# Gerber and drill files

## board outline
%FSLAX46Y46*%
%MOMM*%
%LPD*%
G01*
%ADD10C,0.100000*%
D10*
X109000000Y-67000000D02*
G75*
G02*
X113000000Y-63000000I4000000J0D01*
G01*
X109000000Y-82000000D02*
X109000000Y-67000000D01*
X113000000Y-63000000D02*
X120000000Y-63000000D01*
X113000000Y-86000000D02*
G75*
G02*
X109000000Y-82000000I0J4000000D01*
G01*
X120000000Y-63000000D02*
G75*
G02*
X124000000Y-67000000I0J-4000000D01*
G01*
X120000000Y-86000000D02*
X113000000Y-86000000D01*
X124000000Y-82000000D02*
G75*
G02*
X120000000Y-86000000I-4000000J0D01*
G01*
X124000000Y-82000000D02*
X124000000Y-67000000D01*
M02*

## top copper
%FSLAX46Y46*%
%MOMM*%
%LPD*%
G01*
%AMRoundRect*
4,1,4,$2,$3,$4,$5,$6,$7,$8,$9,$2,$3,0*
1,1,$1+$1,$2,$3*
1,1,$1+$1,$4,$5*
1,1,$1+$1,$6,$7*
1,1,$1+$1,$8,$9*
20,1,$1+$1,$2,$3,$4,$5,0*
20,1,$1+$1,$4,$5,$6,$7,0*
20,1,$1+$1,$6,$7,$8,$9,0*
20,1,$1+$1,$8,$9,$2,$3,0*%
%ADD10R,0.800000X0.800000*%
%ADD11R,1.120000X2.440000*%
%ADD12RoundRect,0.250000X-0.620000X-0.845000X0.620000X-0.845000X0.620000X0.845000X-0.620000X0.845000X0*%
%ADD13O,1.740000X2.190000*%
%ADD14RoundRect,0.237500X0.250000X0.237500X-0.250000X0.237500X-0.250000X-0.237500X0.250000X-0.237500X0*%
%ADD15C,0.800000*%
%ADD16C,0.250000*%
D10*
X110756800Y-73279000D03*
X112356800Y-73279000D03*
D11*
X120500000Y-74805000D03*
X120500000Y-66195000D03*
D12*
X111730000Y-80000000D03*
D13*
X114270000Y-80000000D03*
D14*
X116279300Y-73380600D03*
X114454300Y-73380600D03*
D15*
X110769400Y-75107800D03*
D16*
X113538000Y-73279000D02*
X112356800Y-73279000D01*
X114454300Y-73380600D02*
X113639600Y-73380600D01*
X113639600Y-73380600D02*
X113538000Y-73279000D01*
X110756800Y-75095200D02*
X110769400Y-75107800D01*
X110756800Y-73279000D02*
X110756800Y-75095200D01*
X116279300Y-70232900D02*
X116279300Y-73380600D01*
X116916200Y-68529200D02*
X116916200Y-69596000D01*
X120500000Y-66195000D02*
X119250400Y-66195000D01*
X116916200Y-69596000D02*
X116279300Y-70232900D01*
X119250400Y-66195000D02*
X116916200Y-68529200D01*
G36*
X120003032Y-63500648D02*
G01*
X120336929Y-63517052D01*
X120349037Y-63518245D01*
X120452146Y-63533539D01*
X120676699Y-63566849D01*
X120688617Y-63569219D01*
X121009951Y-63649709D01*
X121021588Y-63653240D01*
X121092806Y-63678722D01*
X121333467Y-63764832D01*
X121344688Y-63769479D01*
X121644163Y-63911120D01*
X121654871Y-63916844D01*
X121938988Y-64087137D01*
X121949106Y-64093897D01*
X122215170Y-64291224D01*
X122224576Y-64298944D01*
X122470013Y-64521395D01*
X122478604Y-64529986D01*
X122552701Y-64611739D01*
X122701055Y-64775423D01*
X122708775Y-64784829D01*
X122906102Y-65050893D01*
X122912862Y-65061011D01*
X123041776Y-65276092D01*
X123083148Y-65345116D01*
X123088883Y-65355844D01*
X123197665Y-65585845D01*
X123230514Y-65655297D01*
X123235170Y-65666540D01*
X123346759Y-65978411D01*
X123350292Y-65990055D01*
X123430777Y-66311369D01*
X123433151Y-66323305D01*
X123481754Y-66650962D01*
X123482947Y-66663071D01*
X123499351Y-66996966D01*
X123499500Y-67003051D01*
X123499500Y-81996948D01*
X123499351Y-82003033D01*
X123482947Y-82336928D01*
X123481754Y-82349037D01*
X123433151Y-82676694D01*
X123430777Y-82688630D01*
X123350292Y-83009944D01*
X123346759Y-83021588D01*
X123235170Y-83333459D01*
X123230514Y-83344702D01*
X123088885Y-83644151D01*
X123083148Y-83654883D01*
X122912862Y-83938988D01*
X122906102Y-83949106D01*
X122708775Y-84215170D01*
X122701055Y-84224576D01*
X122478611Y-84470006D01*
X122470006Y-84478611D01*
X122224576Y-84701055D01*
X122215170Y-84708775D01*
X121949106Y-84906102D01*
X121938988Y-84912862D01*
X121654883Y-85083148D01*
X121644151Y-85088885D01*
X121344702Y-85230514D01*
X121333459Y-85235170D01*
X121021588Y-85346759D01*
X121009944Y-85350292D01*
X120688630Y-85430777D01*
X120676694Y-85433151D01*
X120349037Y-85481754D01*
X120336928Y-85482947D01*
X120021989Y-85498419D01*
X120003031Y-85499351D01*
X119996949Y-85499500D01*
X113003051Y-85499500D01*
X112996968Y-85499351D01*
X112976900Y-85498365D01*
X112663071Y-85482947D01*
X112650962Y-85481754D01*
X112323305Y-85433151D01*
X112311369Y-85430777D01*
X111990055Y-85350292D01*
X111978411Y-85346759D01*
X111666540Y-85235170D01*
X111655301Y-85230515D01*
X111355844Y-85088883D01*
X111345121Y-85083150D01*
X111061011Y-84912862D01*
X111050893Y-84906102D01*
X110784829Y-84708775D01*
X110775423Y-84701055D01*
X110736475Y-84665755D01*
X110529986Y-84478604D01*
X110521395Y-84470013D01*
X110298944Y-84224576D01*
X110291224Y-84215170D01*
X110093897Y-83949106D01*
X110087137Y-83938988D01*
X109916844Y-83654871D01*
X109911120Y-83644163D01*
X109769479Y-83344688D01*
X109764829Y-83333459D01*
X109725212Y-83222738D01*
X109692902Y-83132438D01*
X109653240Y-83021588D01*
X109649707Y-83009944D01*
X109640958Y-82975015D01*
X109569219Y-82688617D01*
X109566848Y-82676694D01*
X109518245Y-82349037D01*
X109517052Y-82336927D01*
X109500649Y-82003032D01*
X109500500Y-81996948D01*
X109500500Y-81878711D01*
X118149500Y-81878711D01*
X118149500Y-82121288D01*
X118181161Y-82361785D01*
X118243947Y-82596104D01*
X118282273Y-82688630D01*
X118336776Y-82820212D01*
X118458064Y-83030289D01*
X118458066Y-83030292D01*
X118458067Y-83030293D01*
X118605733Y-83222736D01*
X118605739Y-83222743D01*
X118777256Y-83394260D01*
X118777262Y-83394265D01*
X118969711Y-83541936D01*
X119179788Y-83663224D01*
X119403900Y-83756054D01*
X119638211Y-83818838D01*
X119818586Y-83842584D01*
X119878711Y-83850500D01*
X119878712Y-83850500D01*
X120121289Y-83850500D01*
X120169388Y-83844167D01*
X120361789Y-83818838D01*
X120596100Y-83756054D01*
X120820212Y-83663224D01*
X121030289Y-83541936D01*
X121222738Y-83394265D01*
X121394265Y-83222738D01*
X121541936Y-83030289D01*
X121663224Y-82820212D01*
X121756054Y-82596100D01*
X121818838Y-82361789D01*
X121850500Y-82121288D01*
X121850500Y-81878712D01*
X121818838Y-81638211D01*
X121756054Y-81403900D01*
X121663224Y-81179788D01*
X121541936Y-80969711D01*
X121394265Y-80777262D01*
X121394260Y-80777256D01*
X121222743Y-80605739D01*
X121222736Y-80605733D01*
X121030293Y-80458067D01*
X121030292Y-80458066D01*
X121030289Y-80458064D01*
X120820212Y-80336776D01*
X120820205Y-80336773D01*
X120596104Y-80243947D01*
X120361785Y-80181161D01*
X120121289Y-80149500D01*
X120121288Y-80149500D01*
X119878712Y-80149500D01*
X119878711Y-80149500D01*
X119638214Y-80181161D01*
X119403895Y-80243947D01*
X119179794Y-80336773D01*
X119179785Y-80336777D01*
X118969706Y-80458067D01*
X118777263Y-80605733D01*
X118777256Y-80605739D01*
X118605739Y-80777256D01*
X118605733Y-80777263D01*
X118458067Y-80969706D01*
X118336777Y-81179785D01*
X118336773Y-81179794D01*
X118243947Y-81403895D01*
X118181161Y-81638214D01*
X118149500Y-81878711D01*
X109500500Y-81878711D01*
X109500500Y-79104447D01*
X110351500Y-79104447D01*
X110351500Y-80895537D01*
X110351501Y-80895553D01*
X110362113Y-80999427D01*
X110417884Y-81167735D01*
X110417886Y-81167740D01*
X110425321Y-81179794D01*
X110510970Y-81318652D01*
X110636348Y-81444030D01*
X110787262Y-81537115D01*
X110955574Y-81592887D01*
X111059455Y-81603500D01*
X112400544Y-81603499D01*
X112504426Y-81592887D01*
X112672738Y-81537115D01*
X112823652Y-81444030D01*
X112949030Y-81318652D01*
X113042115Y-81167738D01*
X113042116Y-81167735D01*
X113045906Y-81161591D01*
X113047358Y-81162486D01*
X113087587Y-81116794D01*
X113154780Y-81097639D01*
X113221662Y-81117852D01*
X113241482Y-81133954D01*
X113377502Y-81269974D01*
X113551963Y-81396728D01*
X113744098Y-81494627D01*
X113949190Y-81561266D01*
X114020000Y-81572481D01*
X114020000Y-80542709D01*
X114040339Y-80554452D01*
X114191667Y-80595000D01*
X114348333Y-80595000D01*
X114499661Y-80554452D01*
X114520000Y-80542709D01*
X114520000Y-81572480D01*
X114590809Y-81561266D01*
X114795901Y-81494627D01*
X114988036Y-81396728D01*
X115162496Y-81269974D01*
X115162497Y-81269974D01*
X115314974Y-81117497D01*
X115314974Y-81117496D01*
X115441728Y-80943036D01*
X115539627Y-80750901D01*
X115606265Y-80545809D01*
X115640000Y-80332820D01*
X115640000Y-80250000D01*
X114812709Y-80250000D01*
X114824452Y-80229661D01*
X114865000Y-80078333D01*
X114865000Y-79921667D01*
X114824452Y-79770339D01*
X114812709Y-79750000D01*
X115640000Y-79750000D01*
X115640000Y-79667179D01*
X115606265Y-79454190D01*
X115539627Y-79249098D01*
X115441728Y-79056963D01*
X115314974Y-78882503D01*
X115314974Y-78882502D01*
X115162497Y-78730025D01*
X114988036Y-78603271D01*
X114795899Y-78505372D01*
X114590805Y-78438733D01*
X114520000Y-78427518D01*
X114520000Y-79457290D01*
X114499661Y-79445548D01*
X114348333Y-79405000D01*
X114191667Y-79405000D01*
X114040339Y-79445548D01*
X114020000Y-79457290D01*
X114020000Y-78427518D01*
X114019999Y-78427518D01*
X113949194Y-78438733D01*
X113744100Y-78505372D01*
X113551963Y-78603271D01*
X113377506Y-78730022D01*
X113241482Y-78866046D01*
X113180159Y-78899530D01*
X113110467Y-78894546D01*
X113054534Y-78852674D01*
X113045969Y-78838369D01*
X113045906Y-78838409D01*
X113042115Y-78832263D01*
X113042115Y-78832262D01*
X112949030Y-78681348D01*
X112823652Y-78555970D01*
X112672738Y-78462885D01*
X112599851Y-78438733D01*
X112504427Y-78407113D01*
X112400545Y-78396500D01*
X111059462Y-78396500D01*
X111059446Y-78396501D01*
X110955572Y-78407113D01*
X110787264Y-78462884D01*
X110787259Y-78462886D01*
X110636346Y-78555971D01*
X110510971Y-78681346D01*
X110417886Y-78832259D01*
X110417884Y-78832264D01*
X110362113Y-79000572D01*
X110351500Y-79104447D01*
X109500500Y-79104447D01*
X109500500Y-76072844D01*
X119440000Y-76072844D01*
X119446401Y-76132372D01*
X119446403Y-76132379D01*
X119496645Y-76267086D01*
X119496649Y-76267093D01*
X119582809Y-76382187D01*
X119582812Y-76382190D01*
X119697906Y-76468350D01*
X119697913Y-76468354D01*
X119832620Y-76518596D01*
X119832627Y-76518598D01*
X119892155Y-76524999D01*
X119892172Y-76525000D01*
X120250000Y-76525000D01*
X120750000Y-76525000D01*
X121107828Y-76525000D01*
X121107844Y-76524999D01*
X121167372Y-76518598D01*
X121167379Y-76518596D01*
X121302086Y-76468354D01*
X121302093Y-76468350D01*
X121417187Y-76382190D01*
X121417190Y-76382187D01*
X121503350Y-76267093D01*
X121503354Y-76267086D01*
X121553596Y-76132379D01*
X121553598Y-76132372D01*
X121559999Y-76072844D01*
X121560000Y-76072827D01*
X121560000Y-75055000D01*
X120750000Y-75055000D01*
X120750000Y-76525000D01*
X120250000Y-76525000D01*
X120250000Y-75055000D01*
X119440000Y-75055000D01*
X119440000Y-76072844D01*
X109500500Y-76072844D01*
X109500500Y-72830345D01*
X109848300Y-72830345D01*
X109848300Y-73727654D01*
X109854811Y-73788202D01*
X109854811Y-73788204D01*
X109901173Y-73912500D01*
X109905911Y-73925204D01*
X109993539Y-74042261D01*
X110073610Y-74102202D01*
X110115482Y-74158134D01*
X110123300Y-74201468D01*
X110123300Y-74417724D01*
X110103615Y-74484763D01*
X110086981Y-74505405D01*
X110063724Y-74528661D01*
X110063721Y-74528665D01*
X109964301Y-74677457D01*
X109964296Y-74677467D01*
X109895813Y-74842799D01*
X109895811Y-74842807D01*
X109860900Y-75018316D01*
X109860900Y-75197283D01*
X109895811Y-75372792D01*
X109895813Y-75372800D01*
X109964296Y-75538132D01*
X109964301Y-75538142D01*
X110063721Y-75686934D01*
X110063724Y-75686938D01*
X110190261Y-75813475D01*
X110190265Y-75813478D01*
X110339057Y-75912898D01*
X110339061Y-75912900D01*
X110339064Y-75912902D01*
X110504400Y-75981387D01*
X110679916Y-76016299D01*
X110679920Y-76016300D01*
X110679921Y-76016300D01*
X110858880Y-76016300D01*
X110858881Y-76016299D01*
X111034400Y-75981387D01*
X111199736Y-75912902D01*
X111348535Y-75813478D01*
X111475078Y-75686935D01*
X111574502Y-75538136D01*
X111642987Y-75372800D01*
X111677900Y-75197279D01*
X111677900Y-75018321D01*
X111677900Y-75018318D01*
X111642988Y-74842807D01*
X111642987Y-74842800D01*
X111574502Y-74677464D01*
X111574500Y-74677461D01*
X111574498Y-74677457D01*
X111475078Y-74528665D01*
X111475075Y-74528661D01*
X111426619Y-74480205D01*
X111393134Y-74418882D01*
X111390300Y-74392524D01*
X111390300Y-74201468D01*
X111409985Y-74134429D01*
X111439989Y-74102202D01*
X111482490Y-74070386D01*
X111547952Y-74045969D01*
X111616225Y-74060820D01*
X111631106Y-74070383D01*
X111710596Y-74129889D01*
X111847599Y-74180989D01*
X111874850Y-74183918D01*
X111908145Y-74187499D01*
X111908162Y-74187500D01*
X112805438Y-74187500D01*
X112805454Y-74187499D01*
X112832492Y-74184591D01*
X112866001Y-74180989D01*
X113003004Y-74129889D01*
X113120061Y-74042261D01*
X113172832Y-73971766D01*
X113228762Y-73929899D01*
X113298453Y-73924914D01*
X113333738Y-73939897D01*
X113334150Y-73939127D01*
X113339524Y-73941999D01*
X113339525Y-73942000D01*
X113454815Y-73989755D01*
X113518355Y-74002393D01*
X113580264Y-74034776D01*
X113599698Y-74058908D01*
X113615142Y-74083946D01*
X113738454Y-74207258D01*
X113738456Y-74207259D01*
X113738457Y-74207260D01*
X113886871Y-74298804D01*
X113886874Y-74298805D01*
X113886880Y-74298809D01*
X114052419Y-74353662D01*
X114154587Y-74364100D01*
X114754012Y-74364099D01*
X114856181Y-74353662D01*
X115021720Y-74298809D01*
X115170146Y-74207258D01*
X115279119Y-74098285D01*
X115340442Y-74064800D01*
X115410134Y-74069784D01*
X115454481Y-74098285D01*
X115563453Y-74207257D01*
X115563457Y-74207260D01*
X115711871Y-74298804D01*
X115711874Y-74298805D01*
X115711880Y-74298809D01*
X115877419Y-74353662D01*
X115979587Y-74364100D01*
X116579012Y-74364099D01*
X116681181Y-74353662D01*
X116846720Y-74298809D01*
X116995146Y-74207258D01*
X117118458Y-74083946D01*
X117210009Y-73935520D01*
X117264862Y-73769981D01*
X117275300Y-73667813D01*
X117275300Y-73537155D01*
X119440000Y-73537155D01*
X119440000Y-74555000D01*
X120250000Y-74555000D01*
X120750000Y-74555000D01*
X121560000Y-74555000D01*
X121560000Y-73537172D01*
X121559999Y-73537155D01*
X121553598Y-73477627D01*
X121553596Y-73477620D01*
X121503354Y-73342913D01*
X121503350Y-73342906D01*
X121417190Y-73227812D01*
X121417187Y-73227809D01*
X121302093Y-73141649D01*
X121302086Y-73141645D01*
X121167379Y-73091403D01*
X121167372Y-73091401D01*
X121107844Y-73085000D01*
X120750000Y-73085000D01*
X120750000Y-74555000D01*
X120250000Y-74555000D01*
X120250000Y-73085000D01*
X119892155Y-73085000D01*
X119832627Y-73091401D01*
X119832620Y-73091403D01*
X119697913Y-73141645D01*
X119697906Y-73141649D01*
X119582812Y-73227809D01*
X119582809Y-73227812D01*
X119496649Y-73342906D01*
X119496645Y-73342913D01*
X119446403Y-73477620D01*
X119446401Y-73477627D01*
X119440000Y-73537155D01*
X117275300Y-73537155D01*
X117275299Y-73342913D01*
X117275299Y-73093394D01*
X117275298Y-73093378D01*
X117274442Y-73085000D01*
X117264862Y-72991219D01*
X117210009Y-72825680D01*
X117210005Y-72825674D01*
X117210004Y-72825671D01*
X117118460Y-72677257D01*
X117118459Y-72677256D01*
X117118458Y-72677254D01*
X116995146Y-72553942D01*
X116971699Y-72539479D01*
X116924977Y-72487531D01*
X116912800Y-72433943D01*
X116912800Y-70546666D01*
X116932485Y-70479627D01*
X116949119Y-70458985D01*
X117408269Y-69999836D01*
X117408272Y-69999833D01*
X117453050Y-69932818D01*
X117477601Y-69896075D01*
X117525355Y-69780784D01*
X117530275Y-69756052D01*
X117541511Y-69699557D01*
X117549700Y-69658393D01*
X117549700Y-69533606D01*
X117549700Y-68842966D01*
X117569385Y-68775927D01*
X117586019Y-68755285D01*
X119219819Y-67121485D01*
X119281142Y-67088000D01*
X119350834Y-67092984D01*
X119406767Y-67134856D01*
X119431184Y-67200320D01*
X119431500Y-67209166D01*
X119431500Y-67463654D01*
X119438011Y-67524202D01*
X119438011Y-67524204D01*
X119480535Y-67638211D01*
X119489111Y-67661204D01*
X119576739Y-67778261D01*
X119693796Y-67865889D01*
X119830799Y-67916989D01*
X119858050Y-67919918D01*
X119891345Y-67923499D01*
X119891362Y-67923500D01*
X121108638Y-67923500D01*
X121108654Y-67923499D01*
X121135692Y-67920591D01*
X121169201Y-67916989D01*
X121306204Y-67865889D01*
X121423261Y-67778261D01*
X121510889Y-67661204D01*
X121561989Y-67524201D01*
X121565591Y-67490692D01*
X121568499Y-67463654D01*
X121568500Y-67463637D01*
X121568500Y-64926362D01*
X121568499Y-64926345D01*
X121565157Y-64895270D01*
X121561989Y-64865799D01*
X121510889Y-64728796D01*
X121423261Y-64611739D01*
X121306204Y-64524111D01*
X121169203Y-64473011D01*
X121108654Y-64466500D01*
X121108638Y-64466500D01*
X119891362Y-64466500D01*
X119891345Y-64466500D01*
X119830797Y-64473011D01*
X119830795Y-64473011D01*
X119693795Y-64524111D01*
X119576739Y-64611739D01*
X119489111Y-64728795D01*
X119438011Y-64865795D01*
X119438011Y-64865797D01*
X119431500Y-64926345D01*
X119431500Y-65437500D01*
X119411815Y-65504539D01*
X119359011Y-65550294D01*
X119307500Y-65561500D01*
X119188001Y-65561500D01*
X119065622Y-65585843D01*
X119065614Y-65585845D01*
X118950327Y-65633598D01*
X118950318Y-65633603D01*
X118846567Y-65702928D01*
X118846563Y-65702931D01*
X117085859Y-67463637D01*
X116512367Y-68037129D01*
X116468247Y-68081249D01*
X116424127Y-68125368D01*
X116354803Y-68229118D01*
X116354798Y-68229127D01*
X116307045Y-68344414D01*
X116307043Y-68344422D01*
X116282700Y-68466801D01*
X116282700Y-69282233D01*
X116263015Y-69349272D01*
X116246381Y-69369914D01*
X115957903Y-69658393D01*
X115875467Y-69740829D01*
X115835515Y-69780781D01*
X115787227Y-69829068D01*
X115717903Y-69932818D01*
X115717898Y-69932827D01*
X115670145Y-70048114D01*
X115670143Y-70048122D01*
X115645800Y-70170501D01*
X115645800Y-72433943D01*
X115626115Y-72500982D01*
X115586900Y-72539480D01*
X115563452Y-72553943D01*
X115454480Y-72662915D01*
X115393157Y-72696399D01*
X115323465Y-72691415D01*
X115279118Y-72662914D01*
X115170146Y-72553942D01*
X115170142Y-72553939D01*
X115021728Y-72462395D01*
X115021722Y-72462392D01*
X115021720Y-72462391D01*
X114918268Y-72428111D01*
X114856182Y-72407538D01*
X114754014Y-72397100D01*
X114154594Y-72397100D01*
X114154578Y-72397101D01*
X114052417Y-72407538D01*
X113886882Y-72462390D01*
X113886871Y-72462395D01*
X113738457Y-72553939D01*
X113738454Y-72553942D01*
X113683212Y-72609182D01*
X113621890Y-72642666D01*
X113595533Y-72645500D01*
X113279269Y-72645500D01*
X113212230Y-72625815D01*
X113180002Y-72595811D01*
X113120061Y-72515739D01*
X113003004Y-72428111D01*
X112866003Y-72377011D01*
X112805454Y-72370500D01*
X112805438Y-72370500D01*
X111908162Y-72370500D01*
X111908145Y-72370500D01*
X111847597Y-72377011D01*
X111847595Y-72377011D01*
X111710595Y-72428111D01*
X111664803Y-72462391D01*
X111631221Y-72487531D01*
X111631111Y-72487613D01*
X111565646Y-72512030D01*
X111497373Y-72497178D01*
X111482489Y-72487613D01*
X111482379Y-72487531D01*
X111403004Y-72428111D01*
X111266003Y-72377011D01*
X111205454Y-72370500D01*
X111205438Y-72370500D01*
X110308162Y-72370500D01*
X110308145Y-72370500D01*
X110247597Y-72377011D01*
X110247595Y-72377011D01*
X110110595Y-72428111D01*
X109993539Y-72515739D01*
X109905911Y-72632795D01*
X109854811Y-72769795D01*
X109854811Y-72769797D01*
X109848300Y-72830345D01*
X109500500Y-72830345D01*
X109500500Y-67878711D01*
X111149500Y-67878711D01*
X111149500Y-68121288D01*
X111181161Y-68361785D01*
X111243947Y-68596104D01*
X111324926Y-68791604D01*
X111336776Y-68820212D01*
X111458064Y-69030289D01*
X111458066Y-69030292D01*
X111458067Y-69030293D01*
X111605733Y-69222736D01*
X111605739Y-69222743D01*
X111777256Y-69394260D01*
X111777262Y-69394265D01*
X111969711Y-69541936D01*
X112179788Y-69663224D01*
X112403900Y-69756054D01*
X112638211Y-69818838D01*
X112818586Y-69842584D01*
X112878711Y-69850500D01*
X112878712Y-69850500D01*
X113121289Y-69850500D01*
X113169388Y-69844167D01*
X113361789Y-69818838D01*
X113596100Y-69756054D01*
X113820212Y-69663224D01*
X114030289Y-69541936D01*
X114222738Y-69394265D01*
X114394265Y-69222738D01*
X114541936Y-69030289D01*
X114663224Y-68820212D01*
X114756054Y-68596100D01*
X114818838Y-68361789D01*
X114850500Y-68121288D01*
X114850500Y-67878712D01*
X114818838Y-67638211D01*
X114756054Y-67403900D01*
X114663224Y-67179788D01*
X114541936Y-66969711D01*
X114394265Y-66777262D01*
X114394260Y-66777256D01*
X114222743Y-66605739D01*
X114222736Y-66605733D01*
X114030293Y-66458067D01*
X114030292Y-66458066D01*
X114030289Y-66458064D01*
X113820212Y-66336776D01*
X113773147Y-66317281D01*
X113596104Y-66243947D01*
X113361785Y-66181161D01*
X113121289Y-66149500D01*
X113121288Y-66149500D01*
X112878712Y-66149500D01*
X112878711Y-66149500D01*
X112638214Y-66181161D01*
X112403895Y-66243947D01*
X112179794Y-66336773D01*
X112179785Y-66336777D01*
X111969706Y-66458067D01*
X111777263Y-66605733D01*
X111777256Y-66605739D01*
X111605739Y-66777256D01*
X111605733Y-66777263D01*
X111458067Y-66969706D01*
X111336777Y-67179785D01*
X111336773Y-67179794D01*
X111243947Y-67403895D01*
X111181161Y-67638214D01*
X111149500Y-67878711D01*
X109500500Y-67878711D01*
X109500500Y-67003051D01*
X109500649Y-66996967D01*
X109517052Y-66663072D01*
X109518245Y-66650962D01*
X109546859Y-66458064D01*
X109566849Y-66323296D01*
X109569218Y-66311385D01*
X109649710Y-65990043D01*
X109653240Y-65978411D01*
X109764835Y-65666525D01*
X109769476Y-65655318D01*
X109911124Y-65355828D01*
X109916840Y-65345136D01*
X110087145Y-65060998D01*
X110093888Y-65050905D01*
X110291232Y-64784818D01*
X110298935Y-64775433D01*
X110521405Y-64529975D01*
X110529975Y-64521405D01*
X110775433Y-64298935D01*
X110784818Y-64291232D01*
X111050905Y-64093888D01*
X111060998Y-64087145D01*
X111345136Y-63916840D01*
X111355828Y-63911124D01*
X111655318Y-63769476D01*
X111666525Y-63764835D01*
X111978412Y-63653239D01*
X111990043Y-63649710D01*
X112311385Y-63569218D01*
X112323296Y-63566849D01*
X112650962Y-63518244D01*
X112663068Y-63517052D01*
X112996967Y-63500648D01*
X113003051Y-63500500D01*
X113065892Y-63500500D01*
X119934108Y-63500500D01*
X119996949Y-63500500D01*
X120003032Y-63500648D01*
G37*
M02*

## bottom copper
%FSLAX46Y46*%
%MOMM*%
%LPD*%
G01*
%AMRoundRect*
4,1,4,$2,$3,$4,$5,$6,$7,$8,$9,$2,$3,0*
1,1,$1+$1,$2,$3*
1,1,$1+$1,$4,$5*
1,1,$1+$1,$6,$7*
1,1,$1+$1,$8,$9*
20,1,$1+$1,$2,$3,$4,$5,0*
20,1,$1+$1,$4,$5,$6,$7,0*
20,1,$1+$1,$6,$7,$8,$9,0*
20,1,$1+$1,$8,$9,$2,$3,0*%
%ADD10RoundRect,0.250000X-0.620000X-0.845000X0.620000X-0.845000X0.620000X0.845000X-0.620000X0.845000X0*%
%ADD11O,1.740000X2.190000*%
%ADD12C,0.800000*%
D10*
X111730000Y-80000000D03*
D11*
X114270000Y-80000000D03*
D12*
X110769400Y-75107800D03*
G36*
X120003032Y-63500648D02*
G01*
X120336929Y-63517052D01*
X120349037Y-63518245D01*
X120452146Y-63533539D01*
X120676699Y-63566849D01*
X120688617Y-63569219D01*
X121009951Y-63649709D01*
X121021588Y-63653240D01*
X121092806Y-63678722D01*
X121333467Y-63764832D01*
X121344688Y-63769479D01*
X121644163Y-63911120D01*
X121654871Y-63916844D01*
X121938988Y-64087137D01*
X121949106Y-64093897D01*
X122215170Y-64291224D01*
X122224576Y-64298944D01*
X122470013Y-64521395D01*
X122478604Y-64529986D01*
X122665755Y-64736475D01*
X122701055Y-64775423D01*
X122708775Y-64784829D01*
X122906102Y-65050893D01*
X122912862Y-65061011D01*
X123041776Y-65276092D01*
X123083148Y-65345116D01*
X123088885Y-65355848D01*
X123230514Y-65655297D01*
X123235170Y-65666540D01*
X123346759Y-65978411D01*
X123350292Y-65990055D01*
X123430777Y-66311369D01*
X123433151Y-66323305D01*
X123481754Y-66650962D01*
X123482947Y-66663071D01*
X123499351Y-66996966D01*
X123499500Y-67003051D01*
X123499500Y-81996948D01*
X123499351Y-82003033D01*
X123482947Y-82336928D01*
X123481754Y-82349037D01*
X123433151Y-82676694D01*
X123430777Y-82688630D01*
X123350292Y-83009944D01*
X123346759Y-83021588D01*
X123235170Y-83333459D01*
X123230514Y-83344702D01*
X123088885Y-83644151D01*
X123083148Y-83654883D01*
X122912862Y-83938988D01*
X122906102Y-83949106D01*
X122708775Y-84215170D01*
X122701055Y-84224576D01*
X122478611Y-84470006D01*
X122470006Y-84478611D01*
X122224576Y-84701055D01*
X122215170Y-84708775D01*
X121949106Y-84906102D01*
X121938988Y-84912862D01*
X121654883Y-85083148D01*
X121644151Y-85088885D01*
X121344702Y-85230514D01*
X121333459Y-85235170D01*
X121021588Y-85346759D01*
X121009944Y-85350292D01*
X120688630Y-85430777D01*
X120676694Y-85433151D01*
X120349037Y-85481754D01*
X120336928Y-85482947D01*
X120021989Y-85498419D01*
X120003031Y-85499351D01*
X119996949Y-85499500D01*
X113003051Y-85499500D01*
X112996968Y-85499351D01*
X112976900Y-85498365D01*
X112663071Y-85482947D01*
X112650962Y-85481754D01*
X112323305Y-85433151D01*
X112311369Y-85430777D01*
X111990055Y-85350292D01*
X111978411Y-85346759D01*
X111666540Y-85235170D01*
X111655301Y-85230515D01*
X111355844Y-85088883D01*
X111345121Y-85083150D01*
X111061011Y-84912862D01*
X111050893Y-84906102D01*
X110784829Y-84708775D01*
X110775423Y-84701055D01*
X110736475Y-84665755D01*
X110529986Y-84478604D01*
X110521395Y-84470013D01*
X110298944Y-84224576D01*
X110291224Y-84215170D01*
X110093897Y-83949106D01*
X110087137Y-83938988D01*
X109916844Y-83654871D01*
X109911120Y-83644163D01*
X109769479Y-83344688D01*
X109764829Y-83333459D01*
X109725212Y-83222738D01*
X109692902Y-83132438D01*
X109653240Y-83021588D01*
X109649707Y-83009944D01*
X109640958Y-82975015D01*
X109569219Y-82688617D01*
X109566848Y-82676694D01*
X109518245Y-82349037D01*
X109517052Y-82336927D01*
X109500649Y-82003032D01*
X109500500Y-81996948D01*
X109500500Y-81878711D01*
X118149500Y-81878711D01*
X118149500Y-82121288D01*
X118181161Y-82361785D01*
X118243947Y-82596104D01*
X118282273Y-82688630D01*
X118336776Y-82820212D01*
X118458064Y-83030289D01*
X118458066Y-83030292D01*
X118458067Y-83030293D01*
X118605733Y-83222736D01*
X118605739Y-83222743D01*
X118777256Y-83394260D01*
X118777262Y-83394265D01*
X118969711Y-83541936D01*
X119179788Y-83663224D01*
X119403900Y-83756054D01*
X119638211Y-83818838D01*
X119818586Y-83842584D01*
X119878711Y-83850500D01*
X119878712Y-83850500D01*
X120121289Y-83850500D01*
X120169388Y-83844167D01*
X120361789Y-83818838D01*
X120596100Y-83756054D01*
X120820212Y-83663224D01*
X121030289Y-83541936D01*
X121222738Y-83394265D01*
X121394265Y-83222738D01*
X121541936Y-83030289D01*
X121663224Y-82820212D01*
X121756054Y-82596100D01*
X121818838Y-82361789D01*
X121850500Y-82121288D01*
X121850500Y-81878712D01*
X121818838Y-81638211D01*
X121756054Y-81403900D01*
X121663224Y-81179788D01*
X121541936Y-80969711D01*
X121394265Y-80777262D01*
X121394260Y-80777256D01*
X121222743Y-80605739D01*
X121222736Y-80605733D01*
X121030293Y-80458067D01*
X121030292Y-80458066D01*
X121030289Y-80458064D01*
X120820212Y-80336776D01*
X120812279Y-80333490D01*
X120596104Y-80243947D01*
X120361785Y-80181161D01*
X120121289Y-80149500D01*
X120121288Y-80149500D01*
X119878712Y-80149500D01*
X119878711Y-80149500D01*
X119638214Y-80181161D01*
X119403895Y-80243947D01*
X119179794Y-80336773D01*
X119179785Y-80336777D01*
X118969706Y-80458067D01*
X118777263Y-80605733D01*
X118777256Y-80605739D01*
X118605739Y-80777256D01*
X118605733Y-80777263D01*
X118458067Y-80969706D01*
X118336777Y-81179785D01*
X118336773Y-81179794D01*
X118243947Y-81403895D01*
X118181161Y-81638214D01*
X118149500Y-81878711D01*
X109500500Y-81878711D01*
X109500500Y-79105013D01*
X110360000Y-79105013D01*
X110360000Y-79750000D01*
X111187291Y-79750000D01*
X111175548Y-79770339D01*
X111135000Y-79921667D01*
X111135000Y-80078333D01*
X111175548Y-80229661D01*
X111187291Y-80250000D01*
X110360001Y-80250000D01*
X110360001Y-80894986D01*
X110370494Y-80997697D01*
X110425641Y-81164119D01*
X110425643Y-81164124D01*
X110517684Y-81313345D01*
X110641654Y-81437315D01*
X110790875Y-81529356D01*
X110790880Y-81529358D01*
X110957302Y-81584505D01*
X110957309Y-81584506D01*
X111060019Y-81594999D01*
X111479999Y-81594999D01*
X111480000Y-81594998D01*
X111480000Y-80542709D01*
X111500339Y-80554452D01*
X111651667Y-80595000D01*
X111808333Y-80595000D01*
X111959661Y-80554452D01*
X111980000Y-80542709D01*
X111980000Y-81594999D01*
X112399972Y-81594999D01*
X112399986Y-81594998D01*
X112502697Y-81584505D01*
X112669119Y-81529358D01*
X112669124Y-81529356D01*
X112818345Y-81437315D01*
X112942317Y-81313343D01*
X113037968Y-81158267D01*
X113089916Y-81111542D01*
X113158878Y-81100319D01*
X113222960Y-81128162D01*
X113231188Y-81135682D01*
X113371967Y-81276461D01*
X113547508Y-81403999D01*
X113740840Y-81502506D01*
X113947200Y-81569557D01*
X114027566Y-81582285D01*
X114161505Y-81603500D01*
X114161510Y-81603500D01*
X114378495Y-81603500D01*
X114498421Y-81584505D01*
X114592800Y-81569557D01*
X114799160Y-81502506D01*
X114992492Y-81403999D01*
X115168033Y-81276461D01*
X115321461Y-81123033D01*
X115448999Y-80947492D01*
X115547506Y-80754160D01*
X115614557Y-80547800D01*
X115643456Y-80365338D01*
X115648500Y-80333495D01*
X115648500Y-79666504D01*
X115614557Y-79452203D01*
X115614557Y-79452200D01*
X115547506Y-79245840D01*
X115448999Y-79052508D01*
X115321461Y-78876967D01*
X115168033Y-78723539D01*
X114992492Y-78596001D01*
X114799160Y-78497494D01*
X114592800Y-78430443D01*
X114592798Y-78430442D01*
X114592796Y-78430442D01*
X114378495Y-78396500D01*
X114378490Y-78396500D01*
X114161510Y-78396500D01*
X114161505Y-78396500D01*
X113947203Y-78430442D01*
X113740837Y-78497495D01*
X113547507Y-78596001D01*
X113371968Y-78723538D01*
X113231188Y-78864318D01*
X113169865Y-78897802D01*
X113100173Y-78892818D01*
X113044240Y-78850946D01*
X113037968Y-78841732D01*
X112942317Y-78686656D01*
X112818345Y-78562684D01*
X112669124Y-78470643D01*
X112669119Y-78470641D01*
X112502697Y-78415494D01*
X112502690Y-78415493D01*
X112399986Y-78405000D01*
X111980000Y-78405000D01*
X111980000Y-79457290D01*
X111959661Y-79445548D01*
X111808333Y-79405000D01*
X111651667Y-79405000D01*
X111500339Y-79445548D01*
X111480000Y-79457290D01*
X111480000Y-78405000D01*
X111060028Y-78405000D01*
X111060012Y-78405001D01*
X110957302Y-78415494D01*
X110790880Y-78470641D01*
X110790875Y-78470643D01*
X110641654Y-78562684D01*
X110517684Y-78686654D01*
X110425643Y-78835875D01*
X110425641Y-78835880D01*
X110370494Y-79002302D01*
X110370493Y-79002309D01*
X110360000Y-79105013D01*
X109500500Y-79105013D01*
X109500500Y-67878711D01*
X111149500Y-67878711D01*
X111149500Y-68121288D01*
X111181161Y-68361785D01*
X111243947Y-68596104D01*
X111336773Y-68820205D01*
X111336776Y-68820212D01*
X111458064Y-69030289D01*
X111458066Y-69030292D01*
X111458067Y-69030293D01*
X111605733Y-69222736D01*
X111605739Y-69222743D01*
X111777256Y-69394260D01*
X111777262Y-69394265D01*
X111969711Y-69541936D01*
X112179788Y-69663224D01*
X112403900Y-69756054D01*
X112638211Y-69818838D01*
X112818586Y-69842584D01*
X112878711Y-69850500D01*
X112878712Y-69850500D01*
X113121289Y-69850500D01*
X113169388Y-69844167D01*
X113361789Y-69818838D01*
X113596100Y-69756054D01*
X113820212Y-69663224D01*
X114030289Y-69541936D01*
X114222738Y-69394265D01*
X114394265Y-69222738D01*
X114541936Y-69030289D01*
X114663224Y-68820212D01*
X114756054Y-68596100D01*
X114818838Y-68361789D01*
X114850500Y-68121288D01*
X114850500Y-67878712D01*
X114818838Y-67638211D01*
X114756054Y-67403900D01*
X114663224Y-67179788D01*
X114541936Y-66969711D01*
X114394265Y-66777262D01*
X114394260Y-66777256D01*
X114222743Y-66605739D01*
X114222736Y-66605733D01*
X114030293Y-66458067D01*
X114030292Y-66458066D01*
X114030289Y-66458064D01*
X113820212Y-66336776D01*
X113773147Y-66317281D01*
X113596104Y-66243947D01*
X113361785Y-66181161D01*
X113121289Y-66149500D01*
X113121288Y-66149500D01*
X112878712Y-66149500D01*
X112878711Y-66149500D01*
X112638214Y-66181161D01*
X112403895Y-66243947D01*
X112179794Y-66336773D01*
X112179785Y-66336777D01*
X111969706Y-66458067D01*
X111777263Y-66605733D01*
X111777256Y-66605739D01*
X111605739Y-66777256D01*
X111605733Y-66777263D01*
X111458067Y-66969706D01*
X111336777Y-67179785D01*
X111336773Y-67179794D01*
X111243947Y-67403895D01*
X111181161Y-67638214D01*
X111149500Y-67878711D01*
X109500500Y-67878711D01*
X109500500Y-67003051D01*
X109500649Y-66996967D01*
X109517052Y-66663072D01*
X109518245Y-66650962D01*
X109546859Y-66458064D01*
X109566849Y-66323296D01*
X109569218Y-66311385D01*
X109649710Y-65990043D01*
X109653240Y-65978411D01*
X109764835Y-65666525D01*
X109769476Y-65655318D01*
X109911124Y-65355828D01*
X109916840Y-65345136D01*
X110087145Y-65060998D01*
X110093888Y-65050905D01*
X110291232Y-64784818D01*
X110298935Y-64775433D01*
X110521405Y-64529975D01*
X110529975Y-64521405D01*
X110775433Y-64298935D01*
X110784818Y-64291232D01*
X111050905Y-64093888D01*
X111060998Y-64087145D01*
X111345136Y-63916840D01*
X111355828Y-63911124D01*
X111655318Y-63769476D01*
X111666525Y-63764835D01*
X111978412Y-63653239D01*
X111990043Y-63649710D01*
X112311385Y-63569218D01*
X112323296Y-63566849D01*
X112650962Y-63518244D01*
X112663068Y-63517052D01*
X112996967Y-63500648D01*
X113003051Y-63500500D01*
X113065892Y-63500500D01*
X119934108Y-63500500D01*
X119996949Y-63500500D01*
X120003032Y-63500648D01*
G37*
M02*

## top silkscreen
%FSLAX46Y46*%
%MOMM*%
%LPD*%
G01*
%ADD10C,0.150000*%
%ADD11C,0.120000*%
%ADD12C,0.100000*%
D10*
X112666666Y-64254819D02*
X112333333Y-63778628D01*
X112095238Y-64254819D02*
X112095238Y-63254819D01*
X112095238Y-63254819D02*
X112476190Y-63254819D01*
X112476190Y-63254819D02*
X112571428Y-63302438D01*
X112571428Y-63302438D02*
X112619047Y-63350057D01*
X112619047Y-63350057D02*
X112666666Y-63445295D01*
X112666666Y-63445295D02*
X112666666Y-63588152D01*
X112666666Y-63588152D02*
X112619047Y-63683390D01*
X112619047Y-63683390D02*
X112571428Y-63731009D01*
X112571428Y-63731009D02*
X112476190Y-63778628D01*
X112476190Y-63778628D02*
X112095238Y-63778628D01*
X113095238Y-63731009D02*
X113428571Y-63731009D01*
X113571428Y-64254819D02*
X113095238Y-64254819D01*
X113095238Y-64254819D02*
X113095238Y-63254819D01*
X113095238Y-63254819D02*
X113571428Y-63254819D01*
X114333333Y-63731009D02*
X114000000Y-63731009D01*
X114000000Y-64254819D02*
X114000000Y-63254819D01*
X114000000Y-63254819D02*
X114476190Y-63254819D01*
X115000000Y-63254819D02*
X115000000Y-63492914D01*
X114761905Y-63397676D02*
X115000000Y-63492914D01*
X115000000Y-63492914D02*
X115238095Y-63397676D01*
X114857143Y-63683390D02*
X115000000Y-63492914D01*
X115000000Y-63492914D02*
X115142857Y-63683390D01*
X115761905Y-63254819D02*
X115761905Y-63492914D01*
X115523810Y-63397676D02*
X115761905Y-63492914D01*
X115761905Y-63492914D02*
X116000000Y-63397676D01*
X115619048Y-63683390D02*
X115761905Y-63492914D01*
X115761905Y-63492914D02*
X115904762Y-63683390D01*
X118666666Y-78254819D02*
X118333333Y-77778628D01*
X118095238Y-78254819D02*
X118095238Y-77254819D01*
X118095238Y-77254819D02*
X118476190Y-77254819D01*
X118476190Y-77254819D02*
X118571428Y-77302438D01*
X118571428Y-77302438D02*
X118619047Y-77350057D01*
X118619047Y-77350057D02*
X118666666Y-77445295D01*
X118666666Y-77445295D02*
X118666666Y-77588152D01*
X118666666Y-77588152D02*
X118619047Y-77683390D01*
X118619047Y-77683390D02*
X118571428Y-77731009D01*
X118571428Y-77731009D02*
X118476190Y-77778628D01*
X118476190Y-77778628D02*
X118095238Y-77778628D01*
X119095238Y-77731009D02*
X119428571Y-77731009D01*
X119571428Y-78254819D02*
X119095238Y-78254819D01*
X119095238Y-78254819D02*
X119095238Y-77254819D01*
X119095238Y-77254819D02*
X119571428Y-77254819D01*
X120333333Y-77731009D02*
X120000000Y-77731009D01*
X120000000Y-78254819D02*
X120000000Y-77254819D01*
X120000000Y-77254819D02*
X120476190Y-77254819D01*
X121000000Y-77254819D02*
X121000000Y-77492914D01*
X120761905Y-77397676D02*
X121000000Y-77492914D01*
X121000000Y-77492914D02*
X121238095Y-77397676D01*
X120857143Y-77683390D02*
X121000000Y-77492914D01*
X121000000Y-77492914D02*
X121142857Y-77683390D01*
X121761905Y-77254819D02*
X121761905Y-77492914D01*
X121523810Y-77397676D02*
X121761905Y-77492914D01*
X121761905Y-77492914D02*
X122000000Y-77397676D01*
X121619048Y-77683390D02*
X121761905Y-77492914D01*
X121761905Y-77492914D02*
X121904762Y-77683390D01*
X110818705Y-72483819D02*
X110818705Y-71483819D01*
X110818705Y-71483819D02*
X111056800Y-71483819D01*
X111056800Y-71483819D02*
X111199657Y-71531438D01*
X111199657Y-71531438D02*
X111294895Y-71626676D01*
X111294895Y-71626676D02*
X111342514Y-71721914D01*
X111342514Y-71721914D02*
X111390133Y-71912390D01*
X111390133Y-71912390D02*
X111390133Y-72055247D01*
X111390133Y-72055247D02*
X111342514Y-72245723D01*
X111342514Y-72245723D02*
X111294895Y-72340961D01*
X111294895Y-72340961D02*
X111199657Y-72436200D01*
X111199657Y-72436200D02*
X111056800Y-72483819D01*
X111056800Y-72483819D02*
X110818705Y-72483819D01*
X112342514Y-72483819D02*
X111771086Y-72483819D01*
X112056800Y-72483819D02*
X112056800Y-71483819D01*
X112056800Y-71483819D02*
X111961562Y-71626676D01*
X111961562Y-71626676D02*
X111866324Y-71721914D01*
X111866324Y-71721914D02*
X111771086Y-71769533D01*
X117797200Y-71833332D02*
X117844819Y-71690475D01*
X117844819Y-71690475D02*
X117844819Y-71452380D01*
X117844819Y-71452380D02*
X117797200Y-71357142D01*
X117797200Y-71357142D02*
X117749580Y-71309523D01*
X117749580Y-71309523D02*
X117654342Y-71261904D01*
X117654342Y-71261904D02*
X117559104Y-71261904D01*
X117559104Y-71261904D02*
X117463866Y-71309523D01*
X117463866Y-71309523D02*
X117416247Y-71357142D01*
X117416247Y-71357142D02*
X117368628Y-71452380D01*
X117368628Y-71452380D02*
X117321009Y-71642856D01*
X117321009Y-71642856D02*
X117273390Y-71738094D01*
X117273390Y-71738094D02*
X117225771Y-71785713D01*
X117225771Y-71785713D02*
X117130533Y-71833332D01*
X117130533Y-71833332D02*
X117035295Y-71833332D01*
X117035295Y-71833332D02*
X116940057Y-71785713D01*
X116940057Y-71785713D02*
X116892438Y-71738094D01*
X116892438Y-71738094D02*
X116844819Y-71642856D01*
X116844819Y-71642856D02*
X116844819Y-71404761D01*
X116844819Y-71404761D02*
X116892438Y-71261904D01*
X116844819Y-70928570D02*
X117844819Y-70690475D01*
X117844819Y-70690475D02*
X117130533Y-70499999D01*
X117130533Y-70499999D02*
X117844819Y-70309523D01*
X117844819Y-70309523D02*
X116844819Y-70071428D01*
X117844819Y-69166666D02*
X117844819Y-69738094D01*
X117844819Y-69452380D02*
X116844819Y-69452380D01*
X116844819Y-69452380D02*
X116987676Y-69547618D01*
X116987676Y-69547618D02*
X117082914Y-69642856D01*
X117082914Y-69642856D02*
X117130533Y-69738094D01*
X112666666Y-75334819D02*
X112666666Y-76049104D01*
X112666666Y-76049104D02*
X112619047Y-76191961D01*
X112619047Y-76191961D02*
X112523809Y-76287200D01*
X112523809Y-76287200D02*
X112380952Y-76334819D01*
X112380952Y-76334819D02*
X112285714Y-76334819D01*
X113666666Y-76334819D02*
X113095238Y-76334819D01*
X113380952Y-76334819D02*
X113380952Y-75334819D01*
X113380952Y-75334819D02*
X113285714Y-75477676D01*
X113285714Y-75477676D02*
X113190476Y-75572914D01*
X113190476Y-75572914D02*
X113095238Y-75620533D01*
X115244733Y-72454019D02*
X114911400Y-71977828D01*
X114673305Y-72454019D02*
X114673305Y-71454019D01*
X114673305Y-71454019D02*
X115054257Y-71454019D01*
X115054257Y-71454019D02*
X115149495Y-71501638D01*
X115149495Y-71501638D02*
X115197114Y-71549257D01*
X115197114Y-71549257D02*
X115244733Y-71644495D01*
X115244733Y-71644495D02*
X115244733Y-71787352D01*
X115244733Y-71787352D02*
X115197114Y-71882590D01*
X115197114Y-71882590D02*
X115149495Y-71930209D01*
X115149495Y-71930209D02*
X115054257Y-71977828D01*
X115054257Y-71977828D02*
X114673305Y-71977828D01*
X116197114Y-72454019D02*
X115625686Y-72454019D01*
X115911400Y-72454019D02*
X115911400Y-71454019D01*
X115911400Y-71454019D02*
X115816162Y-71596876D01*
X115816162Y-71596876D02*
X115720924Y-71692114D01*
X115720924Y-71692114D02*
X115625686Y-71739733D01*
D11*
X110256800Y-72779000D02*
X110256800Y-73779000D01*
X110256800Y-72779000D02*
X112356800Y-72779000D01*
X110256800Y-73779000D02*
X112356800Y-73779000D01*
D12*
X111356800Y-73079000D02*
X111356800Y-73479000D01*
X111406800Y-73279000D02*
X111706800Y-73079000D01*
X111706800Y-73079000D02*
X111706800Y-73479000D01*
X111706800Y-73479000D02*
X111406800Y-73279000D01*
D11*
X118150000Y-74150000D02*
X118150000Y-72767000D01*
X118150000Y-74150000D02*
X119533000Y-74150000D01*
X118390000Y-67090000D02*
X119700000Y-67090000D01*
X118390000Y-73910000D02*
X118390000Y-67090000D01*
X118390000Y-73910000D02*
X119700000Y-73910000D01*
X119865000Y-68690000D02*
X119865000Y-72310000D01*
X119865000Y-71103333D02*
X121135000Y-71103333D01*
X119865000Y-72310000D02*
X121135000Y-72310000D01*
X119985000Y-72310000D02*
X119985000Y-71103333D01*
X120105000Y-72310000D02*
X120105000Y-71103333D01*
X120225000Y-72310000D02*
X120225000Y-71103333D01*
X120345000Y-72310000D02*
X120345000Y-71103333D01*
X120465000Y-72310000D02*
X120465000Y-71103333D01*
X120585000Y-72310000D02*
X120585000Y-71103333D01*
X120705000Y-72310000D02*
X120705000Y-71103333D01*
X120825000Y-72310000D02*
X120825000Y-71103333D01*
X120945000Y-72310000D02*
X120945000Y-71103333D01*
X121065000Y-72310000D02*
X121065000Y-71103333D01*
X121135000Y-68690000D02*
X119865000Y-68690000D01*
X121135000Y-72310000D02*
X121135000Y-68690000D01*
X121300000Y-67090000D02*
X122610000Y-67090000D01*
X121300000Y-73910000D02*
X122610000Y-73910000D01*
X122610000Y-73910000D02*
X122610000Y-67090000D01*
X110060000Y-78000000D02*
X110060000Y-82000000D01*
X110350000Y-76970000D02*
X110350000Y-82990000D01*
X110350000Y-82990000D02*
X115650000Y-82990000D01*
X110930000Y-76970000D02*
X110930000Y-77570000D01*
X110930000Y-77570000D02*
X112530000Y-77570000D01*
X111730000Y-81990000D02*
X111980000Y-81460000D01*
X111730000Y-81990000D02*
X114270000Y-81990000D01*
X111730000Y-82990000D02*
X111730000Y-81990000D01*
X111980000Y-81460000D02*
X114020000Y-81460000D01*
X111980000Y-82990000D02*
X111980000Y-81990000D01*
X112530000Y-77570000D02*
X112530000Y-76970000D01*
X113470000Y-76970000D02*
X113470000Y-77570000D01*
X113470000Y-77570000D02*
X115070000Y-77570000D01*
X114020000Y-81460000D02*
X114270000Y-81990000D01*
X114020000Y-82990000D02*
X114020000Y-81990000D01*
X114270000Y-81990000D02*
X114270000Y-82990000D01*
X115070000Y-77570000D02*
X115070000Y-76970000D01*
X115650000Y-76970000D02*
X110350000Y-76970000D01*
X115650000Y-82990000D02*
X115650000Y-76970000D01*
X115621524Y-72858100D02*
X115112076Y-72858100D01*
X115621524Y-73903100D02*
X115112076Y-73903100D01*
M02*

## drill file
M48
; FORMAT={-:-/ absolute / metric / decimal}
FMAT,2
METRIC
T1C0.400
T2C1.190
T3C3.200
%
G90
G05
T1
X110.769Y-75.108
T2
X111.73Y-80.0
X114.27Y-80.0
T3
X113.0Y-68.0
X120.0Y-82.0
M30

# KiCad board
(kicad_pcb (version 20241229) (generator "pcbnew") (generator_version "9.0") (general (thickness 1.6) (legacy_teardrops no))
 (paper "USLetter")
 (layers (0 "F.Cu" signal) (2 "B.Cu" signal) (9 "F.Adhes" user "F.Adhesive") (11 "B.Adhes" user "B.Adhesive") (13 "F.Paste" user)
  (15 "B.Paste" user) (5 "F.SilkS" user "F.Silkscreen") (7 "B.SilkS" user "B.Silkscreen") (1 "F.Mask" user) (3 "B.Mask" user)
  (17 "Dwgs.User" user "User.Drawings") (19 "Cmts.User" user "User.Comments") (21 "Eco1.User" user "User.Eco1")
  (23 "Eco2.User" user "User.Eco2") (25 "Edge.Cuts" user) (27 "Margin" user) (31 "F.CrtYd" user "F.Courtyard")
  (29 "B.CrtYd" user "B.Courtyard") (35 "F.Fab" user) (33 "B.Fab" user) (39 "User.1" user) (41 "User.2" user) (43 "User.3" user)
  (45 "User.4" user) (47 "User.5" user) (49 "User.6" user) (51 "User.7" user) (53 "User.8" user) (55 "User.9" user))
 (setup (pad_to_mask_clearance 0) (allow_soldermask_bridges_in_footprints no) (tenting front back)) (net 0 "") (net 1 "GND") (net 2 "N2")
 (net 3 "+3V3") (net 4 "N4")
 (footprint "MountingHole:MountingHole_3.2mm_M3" (layer "F.Cu") (at 113 68)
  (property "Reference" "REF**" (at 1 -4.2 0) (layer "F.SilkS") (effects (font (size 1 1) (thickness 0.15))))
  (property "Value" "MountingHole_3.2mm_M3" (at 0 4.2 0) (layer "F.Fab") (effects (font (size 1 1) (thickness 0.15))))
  (pad "" np_thru_hole circle (at 0 0) (size 3.2 3.2) (drill 3.2) (layers "*.Cu" "*.Mask")))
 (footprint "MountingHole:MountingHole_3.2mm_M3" (layer "F.Cu") (at 120 82)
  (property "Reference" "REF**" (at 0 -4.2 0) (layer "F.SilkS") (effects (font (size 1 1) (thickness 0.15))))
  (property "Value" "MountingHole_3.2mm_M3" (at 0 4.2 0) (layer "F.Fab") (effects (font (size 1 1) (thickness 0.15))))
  (pad "" np_thru_hole circle (at 0 0) (size 3.2 3.2) (drill 3.2) (layers "*.Cu" "*.Mask")))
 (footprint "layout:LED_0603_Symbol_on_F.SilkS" (layer "F.Cu") (at 111.5568 73.279)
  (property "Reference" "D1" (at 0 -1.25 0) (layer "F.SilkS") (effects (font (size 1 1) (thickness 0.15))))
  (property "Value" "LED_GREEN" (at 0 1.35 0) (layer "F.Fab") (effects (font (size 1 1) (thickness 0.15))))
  (fp_line (start -1.3 -0.5) (end -1.3 0.5) (stroke (width 0.12) (type solid)) (layer "F.SilkS"))
  (fp_line (start -1.3 -0.5) (end 0.8 -0.5) (stroke (width 0.12) (type solid)) (layer "F.SilkS"))
  (fp_line (start -1.3 0.5) (end 0.8 0.5) (stroke (width 0.12) (type solid)) (layer "F.SilkS"))
  (fp_line (start -0.2 -0.2) (end -0.2 0.2) (stroke (width 0.1) (type solid)) (layer "F.SilkS"))
  (fp_line (start -0.15 0) (end 0.15 -0.2) (stroke (width 0.1) (type solid)) (layer "F.SilkS"))
  (fp_line (start 0.15 -0.2) (end 0.15 0.2) (stroke (width 0.1) (type solid)) (layer "F.SilkS"))
  (fp_line (start 0.15 0.2) (end -0.15 0) (stroke (width 0.1) (type solid)) (layer "F.SilkS"))
  (pad "1" smd rect (at -0.8 0 180) (size 0.8 0.8) (layers "F.Cu" "F.Mask" "F.Paste") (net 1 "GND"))
  (pad "2" smd rect (at 0.8 0 180) (size 0.8 0.8) (layers "F.Cu" "F.Mask" "F.Paste") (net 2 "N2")))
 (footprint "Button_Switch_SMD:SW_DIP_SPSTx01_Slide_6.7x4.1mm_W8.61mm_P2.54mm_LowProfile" (layer "F.Cu") (at 120.5 70.5 90)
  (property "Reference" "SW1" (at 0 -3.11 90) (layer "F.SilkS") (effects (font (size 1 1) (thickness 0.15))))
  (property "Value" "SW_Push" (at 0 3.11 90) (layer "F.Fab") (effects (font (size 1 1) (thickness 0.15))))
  (fp_line (start -3.65 -2.35) (end -2.267 -2.35) (stroke (width 0.12) (type solid)) (layer "F.SilkS"))
  (fp_line (start -3.65 -2.35) (end -3.65 -0.967) (stroke (width 0.12) (type solid)) (layer "F.SilkS"))
  (fp_line (start 3.41 -2.11) (end 3.41 -0.8) (stroke (width 0.12) (type solid)) (layer "F.SilkS"))
  (fp_line (start -3.41 -2.11) (end 3.41 -2.11) (stroke (width 0.12) (type solid)) (layer "F.SilkS"))
  (fp_line (start -3.41 -2.11) (end -3.41 -0.8) (stroke (width 0.12) (type solid)) (layer "F.SilkS"))
  (fp_line (start 1.81 -0.635) (end -1.81 -0.635) (stroke (width 0.12) (type solid)) (layer "F.SilkS"))
  (fp_line (start -0.603333 -0.635) (end -0.603333 0.635) (stroke (width 0.12) (type solid)) (layer "F.SilkS"))
  (fp_line (start -1.81 -0.635) (end -1.81 0.635) (stroke (width 0.12) (type solid)) (layer "F.SilkS"))
  (fp_line (start -1.81 -0.515) (end -0.603333 -0.515) (stroke (width 0.12) (type solid)) (layer "F.SilkS"))
  (fp_line (start -1.81 -0.395) (end -0.603333 -0.395) (stroke (width 0.12) (type solid)) (layer "F.SilkS"))
  (fp_line (start -1.81 -0.275) (end -0.603333 -0.275) (stroke (width 0.12) (type solid)) (layer "F.SilkS"))
  (fp_line (start -1.81 -0.155) (end -0.603333 -0.155) (stroke (width 0.12) (type solid)) (layer "F.SilkS"))
  (fp_line (start -1.81 -0.035) (end -0.603333 -0.035) (stroke (width 0.12) (type solid)) (layer "F.SilkS"))
  (fp_line (start -1.81 0.085) (end -0.603333 0.085) (stroke (width 0.12) (type solid)) (layer "F.SilkS"))
  (fp_line (start -1.81 0.205) (end -0.603333 0.205) (stroke (width 0.12) (type solid)) (layer "F.SilkS"))
  (fp_line (start -1.81 0.325) (end -0.603333 0.325) (stroke (width 0.12) (type solid)) (layer "F.SilkS"))
  (fp_line (start -1.81 0.445) (end -0.603333 0.445) (stroke (width 0.12) (type solid)) (layer "F.SilkS"))
  (fp_line (start -1.81 0.565) (end -0.603333 0.565) (stroke (width 0.12) (type solid)) (layer "F.SilkS"))
  (fp_line (start 1.81 0.635) (end 1.81 -0.635) (stroke (width 0.12) (type solid)) (layer "F.SilkS"))
  (fp_line (start -1.81 0.635) (end 1.81 0.635) (stroke (width 0.12) (type solid)) (layer "F.SilkS"))
  (fp_line (start 3.41 0.8) (end 3.41 2.11) (stroke (width 0.12) (type solid)) (layer "F.SilkS"))
  (fp_line (start -3.41 0.8) (end -3.41 2.11) (stroke (width 0.12) (type solid)) (layer "F.SilkS"))
  (fp_line (start -3.41 2.11) (end 3.41 2.11) (stroke (width 0.12) (type solid)) (layer "F.SilkS"))
  (pad "1" smd rect (at -4.305 0 90) (size 2.44 1.12) (layers "F.Cu" "F.Mask" "F.Paste") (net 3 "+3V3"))
  (pad "2" smd rect (at 4.305 0 90) (size 2.44 1.12) (layers "F.Cu" "F.Mask" "F.Paste") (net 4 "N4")))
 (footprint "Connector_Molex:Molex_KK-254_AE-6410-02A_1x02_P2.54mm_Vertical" (layer "F.Cu") (at 111.73 80)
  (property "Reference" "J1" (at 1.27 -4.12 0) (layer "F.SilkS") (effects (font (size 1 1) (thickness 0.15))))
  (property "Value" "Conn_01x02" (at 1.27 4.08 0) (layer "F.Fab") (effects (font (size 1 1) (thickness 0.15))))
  (fp_line (start -1.67 -2) (end -1.67 2) (stroke (width 0.12) (type solid)) (layer "F.SilkS"))
  (fp_line (start -1.38 -3.03) (end -1.38 2.99) (stroke (width 0.12) (type solid)) (layer "F.SilkS"))
  (fp_line (start -1.38 2.99) (end 3.92 2.99) (stroke (width 0.12) (type solid)) (layer "F.SilkS"))
  (fp_line (start -0.8 -3.03) (end -0.8 -2.43) (stroke (width 0.12) (type solid)) (layer "F.SilkS"))
  (fp_line (start -0.8 -2.43) (end 0.8 -2.43) (stroke (width 0.12) (type solid)) (layer "F.SilkS"))
  (fp_line (start 0 1.99) (end 0.25 1.46) (stroke (width 0.12) (type solid)) (layer "F.SilkS"))
  (fp_line (start 0 1.99) (end 2.54 1.99) (stroke (width 0.12) (type solid)) (layer "F.SilkS"))
  (fp_line (start 0 2.99) (end 0 1.99) (stroke (width 0.12) (type solid)) (layer "F.SilkS"))
  (fp_line (start 0.25 1.46) (end 2.29 1.46) (stroke (width 0.12) (type solid)) (layer "F.SilkS"))
  (fp_line (start 0.25 2.99) (end 0.25 1.99) (stroke (width 0.12) (type solid)) (layer "F.SilkS"))
  (fp_line (start 0.8 -2.43) (end 0.8 -3.03) (stroke (width 0.12) (type solid)) (layer "F.SilkS"))
  (fp_line (start 1.74 -3.03) (end 1.74 -2.43) (stroke (width 0.12) (type solid)) (layer "F.SilkS"))
  (fp_line (start 1.74 -2.43) (end 3.34 -2.43) (stroke (width 0.12) (type solid)) (layer "F.SilkS"))
  (fp_line (start 2.29 1.46) (end 2.54 1.99) (stroke (width 0.12) (type solid)) (layer "F.SilkS"))
  (fp_line (start 2.29 2.99) (end 2.29 1.99) (stroke (width 0.12) (type solid)) (layer "F.SilkS"))
  (fp_line (start 2.54 1.99) (end 2.54 2.99) (stroke (width 0.12) (type solid)) (layer "F.SilkS"))
  (fp_line (start 3.34 -2.43) (end 3.34 -3.03) (stroke (width 0.12) (type solid)) (layer "F.SilkS"))
  (fp_line (start 3.92 -3.03) (end -1.38 -3.03) (stroke (width 0.12) (type solid)) (layer "F.SilkS"))
  (fp_line (start 3.92 2.99) (end 3.92 -3.03) (stroke (width 0.12) (type solid)) (layer "F.SilkS"))
  (pad "1" thru_hole roundrect (at 0 0) (size 1.74 2.19) (drill 1.19) (layers "*.Cu" "*.Mask") (remove_unused_layers no)
   (roundrect_rratio 0.143678) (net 1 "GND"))
  (pad "2" thru_hole oval (at 2.54 0) (size 1.74 2.19) (drill 1.19) (layers "*.Cu" "*.Mask") (remove_unused_layers no) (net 3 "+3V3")))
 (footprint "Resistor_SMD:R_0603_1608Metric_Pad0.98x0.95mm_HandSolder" (layer "F.Cu") (at 115.3668 73.3806 180)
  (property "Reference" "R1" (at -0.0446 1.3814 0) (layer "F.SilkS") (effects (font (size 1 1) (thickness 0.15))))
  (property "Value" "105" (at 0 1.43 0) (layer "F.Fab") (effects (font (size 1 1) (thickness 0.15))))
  (fp_line (start -0.254724 0.5225) (end 0.254724 0.5225) (stroke (width 0.12) (type solid)) (layer "F.SilkS"))
  (fp_line (start -0.254724 -0.5225) (end 0.254724 -0.5225) (stroke (width 0.12) (type solid)) (layer "F.SilkS"))
  (pad "1" smd roundrect (at -0.9125 0 180) (size 0.975 0.95) (layers "F.Cu" "F.Mask" "F.Paste") (roundrect_rratio 0.25) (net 4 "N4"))
  (pad "2" smd roundrect (at 0.9125 0 180) (size 0.975 0.95) (layers "F.Cu" "F.Mask" "F.Paste") (roundrect_rratio 0.25) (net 2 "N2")))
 (gr_arc (start 109 67) (mid 110.171573 64.171573) (end 113 63) (stroke (width 0.1) (type default)) (layer "Edge.Cuts"))
 (gr_line (start 109 82) (end 109 67) (stroke (width 0.1) (type default)) (layer "Edge.Cuts"))
 (gr_line (start 113 63) (end 120 63) (stroke (width 0.1) (type default)) (layer "Edge.Cuts"))
 (gr_arc (start 113 86) (mid 110.171573 84.828427) (end 109 82) (stroke (width 0.1) (type default)) (layer "Edge.Cuts"))
 (gr_arc (start 120 63) (mid 122.828427 64.171573) (end 124 67) (stroke (width 0.1) (type default)) (layer "Edge.Cuts"))
 (gr_line (start 120 86) (end 113 86) (stroke (width 0.1) (type default)) (layer "Edge.Cuts"))
 (gr_arc (start 124 82) (mid 122.828427 84.828427) (end 120 86) (stroke (width 0.1) (type default)) (layer "Edge.Cuts"))
 (gr_line (start 124 82) (end 124 67) (stroke (width 0.1) (type default)) (layer "Edge.Cuts"))
 (segment (start 113.538 73.279) (end 112.3568 73.279) (width 0.25) (layer "F.Cu") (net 2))
 (segment (start 114.4543 73.3806) (end 113.6396 73.3806) (width 0.25) (layer "F.Cu") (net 2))
 (segment (start 113.6396 73.3806) (end 113.538 73.279) (width 0.25) (layer "F.Cu") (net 2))
 (segment (start 110.7568 75.0952) (end 110.7694 75.1078) (width 0.25) (layer "F.Cu") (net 1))
 (segment (start 110.7568 73.279) (end 110.7568 75.0952) (width 0.25) (layer "F.Cu") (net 1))
 (via (at 110.7694 75.1078) (size 0.8) (drill 0.4) (layers "F.Cu" "B.Cu") (free yes) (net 1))
 (segment (start 116.2793 70.2329) (end 116.2793 73.3806) (width 0.25) (layer "F.Cu") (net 4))
 (segment (start 116.9162 68.5292) (end 116.9162 69.596) (width 0.25) (layer "F.Cu") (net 4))
 (segment (start 120.5 66.195) (end 119.2504 66.195) (width 0.25) (layer "F.Cu") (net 4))
 (segment (start 116.9162 69.596) (end 116.2793 70.2329) (width 0.25) (layer "F.Cu") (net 4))
 (segment (start 119.2504 66.195) (end 116.9162 68.5292) (width 0.25) (layer "F.Cu") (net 4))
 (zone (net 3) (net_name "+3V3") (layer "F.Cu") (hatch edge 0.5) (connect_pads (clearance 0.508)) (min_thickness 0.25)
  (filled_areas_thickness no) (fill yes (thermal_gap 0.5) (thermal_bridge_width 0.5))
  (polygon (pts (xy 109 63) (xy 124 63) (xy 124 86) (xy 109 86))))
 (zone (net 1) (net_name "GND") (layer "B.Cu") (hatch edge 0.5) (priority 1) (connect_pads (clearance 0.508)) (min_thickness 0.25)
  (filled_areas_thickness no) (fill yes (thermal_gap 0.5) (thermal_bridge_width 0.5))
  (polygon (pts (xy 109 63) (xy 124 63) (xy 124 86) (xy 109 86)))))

